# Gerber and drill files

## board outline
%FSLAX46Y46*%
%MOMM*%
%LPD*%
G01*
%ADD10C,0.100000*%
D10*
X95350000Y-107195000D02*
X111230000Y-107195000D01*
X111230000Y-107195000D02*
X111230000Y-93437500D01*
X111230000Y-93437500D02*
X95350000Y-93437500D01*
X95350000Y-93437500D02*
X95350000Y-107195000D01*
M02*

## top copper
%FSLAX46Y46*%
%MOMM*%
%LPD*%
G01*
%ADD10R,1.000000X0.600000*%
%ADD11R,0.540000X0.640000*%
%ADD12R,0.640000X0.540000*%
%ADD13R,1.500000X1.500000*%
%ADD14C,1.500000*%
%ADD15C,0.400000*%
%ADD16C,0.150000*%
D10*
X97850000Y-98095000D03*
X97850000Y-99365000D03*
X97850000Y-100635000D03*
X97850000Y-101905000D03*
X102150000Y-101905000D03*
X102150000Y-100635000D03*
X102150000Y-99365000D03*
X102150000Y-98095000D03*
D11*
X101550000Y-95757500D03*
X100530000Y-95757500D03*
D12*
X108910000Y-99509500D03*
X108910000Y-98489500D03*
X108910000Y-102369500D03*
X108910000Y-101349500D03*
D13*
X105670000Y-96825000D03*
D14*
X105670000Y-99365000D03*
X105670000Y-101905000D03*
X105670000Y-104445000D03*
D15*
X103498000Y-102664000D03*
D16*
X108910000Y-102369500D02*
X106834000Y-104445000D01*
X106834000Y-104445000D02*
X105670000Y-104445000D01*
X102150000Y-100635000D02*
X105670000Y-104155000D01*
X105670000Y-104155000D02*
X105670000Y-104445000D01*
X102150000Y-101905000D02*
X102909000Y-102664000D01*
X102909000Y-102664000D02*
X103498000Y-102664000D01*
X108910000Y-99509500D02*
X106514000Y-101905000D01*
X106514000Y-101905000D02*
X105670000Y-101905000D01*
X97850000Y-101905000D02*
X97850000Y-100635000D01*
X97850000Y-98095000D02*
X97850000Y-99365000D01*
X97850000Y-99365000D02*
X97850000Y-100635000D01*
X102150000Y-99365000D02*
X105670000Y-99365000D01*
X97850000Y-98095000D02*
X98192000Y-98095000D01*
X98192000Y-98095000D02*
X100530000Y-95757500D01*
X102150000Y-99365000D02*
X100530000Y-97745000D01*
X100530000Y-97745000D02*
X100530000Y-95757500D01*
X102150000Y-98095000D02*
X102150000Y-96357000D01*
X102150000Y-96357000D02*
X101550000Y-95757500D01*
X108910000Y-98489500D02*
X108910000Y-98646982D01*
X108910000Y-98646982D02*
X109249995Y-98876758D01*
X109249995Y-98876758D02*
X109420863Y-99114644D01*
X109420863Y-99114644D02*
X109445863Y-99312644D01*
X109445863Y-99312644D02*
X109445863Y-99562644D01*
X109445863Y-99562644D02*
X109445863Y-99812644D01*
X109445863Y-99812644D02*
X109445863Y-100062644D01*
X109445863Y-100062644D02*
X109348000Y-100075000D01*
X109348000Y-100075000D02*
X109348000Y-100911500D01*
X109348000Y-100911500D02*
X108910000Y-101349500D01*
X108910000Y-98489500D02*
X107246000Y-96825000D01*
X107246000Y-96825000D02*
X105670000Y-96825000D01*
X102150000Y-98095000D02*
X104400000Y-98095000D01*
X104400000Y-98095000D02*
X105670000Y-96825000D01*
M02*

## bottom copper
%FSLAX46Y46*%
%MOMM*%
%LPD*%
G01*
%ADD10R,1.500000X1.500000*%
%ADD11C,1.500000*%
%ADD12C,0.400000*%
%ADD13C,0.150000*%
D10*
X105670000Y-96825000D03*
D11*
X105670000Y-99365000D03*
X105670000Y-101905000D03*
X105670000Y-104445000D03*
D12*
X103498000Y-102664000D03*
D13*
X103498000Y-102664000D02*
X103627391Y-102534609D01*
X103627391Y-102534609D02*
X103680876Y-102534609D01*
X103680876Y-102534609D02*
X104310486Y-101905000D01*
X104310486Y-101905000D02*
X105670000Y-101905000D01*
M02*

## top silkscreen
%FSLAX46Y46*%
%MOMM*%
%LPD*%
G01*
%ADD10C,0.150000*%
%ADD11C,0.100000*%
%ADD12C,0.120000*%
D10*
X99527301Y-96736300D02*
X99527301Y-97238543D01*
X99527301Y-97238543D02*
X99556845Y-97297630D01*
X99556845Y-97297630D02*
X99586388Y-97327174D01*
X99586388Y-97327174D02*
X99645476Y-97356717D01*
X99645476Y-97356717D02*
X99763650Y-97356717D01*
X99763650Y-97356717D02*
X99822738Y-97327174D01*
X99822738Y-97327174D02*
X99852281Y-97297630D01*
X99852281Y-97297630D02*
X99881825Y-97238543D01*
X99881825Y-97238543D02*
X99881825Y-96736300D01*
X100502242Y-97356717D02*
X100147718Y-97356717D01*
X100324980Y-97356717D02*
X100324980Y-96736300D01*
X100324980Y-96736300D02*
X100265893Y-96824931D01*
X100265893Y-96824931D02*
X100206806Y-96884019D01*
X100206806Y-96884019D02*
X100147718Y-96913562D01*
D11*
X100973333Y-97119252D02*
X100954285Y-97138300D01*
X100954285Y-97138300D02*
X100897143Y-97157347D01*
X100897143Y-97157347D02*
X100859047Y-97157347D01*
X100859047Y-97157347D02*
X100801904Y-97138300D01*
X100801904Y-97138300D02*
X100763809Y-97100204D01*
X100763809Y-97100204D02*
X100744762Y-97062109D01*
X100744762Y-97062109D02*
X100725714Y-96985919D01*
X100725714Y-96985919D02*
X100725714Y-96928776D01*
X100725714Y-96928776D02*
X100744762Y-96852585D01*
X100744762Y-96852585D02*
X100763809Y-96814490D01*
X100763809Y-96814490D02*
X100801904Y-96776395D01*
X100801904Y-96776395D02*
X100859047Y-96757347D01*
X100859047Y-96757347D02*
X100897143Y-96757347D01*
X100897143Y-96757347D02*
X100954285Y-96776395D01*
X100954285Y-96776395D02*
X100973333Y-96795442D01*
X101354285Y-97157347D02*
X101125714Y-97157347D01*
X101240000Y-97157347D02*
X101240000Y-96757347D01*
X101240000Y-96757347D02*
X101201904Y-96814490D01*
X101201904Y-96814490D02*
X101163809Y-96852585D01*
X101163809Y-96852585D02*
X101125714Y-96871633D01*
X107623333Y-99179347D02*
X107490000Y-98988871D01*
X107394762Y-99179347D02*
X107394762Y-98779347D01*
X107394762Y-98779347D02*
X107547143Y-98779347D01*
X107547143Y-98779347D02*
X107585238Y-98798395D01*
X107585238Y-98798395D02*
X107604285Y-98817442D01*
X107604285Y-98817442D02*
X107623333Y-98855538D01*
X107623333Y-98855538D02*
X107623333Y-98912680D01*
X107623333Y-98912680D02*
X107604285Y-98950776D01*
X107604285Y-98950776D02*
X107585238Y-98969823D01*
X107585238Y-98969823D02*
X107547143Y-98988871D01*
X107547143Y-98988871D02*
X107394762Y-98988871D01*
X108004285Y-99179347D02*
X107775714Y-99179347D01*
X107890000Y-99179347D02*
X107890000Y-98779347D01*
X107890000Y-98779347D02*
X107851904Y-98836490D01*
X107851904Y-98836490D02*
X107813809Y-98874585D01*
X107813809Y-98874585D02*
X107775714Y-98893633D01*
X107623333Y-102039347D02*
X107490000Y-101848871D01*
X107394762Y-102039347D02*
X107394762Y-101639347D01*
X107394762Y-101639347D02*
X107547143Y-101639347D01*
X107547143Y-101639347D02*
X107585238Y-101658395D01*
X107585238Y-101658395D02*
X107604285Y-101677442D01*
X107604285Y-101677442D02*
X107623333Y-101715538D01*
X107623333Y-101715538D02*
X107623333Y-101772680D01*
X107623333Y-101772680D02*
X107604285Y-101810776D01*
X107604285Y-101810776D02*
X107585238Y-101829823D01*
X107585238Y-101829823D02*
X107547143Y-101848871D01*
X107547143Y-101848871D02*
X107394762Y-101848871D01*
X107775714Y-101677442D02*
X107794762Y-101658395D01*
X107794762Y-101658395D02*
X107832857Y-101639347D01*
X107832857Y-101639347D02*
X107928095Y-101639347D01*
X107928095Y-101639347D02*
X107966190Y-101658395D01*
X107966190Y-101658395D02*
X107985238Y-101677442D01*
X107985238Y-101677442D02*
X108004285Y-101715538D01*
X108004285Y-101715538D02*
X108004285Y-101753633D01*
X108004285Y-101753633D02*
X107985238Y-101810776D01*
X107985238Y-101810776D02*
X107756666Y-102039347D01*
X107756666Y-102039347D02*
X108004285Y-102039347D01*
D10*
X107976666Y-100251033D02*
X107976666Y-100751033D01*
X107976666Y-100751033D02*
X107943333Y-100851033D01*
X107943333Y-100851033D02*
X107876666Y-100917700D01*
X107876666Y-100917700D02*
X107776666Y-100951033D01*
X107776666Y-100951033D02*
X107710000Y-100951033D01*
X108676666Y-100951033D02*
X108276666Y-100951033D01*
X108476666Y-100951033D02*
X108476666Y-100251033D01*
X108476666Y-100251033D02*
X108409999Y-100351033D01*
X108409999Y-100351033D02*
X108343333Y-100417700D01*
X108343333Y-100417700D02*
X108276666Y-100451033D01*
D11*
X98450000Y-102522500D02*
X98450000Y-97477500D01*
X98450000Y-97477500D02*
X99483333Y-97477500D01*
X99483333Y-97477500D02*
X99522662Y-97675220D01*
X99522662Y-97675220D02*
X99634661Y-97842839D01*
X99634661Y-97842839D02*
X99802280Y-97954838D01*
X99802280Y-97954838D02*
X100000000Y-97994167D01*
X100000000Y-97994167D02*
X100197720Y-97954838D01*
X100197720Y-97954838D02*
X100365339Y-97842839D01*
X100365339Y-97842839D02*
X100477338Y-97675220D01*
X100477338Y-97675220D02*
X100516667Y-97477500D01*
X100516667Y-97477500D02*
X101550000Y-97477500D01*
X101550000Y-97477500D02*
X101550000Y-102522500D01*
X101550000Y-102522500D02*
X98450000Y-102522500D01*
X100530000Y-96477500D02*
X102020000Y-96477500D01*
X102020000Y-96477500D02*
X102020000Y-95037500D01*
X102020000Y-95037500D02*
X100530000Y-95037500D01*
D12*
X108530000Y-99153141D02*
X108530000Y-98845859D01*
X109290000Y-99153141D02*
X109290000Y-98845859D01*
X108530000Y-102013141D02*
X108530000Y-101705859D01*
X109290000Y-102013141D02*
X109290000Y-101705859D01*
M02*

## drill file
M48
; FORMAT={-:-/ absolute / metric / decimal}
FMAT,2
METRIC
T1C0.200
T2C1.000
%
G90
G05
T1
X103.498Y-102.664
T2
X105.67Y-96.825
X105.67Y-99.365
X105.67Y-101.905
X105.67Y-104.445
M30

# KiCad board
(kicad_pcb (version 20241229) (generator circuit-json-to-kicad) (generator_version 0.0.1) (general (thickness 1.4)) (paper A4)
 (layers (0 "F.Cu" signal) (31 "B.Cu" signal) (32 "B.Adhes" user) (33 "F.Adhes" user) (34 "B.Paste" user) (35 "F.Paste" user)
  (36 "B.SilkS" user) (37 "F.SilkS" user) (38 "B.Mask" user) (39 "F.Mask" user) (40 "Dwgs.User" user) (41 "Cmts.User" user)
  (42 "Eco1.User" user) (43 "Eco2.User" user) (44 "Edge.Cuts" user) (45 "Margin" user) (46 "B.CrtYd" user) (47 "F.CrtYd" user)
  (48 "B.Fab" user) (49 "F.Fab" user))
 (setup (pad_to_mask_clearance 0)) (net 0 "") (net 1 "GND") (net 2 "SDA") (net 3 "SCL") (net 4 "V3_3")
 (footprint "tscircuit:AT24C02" (layer F.Cu) (at 100 100 0)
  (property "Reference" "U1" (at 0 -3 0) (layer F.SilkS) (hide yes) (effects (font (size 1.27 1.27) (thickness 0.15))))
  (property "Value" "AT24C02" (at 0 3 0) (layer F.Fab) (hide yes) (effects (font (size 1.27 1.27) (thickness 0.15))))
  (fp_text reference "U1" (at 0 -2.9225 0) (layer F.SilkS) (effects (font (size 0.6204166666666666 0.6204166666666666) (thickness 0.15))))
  (fp_line (start -1.5499999999999998 2.5225) (end -1.5499999999999998 -2.5225) (stroke (width 0.1) (type default)) (layer F.SilkS))
  (fp_line (start -1.5499999999999998 -2.5225) (end -0.5166666666666666 -2.5225) (stroke (width 0.1) (type default)) (layer F.SilkS))
  (fp_line (start -0.5166666666666666 -2.5225) (end -0.47733775846416476 -2.32478022661137) (stroke (width 0.1) (type default))
   (layer F.SilkS))
  (fp_line (start -0.47733775846416476 -2.32478022661137) (end -0.3653385036130495 -2.1571614963869505) (stroke (width 0.1) (type default))
   (layer F.SilkS))
  (fp_line (start -0.3653385036130495 -2.1571614963869505) (end -0.19771977338862967 -2.0451622415358353)
   (stroke (width 0.1) (type default)) (layer F.SilkS))
  (fp_line (start -0.19771977338862967 -2.0451622415358353) (end 3.1636708977973285e-17 -2.0058333333333334)
   (stroke (width 0.1) (type default)) (layer F.SilkS))
  (fp_line (start 3.1636708977973285e-17 -2.0058333333333334) (end 0.1977197733886297 -2.0451622415358353)
   (stroke (width 0.1) (type default)) (layer F.SilkS))
  (fp_line (start 0.1977197733886297 -2.0451622415358353) (end 0.3653385036130496 -2.1571614963869505) (stroke (width 0.1) (type default))
   (layer F.SilkS))
  (fp_line (start 0.3653385036130496 -2.1571614963869505) (end 0.47733775846416476 -2.32478022661137) (stroke (width 0.1) (type default))
   (layer F.SilkS))
  (fp_line (start 0.47733775846416476 -2.32478022661137) (end 0.5166666666666666 -2.5225) (stroke (width 0.1) (type default))
   (layer F.SilkS))
  (fp_line (start 0.5166666666666666 -2.5225) (end 1.5499999999999998 -2.5225) (stroke (width 0.1) (type default)) (layer F.SilkS))
  (fp_line (start 1.5499999999999998 -2.5225) (end 1.5499999999999998 2.5225) (stroke (width 0.1) (type default)) (layer F.SilkS))
  (fp_line (start 1.5499999999999998 2.5225) (end -1.5499999999999998 2.5225) (stroke (width 0.1) (type default)) (layer F.SilkS))
  (pad "1" smd rect (at -2.15 -1.905 0) (size 1 0.6) (layers F.Cu F.Paste F.Mask) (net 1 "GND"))
  (pad "2" smd rect (at -2.15 -0.635 0) (size 1 0.6) (layers F.Cu F.Paste F.Mask) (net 1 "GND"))
  (pad "3" smd rect (at -2.15 0.635 0) (size 1 0.6) (layers F.Cu F.Paste F.Mask) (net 1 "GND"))
  (pad "4" smd rect (at -2.15 1.905 0) (size 1 0.6) (layers F.Cu F.Paste F.Mask) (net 1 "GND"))
  (pad "5" smd rect (at 2.15 1.905 0) (size 1 0.6) (layers F.Cu F.Paste F.Mask) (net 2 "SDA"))
  (pad "6" smd rect (at 2.15 0.635 0) (size 1 0.6) (layers F.Cu F.Paste F.Mask) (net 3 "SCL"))
  (pad "7" smd rect (at 2.15 -0.635 0) (size 1 0.6) (layers F.Cu F.Paste F.Mask) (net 1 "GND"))
  (pad "8" smd rect (at 2.15 -1.905 0) (size 1 0.6) (layers F.Cu F.Paste F.Mask) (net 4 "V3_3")))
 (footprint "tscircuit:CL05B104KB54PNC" (layer F.Cu) (at 101.04 95.7575 180)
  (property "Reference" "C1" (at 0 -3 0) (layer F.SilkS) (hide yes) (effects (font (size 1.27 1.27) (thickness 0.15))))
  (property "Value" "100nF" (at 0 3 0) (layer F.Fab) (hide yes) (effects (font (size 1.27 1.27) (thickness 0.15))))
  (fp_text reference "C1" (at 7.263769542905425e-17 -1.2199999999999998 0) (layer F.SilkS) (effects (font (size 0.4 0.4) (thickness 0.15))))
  (fp_line (start 0.51 -0.7199999999999999) (end -0.9800000000000001 -0.7200000000000001) (stroke (width 0.1) (type default))
   (layer F.SilkS))
  (fp_line (start -0.9800000000000001 -0.7200000000000001) (end -0.9799999999999999 0.7199999999999999) (stroke (width 0.1) (type default))
   (layer F.SilkS))
  (fp_line (start -0.9799999999999999 0.7199999999999999) (end 0.51 0.7199999999999996) (stroke (width 0.1) (type default)) (layer F.SilkS))
  (pad "1" smd rect (at -0.51 0 0) (size 0.54 0.64) (layers F.Cu F.Paste F.Mask) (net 4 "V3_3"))
  (pad "2" smd rect (at 0.5100000000000001 0 0) (size 0.54 0.64) (layers F.Cu F.Paste F.Mask) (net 1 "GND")))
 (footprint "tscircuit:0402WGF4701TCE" (layer F.Cu) (at 108.91 98.9995 90)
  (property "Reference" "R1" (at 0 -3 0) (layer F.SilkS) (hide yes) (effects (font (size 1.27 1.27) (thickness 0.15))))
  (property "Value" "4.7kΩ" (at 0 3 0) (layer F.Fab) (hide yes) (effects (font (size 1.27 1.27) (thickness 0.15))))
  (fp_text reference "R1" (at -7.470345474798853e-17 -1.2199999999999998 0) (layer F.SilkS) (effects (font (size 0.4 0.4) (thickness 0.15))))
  (fp_line (start -0.15364099999999994 -0.3800000000000008) (end 0.1536409999999999 -0.3800000000000008)
   (stroke (width 0.12) (type default)) (layer F.SilkS))
  (fp_line (start -0.153641 0.3800000000000008) (end 0.15364099999999994 0.3800000000000008) (stroke (width 0.12) (type default))
   (layer F.SilkS))
  (pad "1" smd rect (at -0.5099999999999999 0 0) (size 0.64 0.54) (layers F.Cu F.Paste F.Mask) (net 2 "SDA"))
  (pad "2" smd rect (at 0.51 0 0) (size 0.64 0.54) (layers F.Cu F.Paste F.Mask) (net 4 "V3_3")))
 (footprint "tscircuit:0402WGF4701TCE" (layer F.Cu) (at 108.91 101.8595 90)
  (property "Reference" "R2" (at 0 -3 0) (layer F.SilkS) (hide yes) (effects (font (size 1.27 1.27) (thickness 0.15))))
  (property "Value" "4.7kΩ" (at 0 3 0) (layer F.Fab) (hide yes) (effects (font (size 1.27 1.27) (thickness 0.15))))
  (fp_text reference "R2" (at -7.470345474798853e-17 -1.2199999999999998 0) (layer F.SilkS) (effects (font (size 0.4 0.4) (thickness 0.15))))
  (fp_line (start -0.15364099999999994 -0.3800000000000008) (end 0.1536409999999999 -0.3800000000000008)
   (stroke (width 0.12) (type default)) (layer F.SilkS))
  (fp_line (start -0.1536409999999999 0.3800000000000008) (end 0.15364099999999994 0.3800000000000008) (stroke (width 0.12) (type default))
   (layer F.SilkS))
  (pad "1" smd rect (at -0.5099999999999998 0 0) (size 0.64 0.54) (layers F.Cu F.Paste F.Mask) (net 3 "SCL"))
  (pad "2" smd rect (at 0.51 0 0) (size 0.64 0.54) (layers F.Cu F.Paste F.Mask) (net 4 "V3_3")))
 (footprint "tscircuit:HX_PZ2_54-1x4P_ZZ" (layer F.Cu) (at 105.67 100.635 -90.00000000000001)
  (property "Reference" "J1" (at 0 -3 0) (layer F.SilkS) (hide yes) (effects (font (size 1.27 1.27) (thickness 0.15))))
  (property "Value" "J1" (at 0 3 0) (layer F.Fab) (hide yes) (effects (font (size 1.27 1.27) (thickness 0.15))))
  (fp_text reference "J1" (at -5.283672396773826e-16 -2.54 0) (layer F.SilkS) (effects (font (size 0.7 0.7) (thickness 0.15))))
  (pad "1" thru_hole rect (at -3.81 5.705062545910424e-16 0) (size 1.5 1.5) (drill 1) (layers *.Cu *.Mask) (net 4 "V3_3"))
  (pad "2" thru_hole circle (at -1.27 4.862282247637226e-16 0) (size 1.5 1.5) (drill 1) (layers *.Cu *.Mask) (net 1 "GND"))
  (pad "3" thru_hole circle (at 1.27 -4.862282247637226e-16 0) (size 1.5 1.5) (drill 1) (layers *.Cu *.Mask) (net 2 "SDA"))
  (pad "4" thru_hole circle (at 3.8100000000000005 -5.705062545910426e-16 0) (size 1.5 1.5) (drill 1) (layers *.Cu *.Mask) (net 3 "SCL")))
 (segment (start 108.91 102.3695) (end 106.834 104.44500000000001) (width 0.15) (layer F.Cu) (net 3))
 (segment (start 106.834 104.44500000000001) (end 105.67 104.44500000000001) (width 0.15) (layer F.Cu) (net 3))
 (segment (start 102.15 100.635) (end 105.67 104.155) (width 0.15) (layer F.Cu) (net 3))
 (segment (start 105.67 104.155) (end 105.67 104.44500000000001) (width 0.15) (layer F.Cu) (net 3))
 (segment (start 102.15 101.905) (end 102.909 102.664) (width 0.15) (layer F.Cu) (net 2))
 (segment (start 102.909 102.664) (end 103.498 102.664) (width 0.15) (layer F.Cu) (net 2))
 (segment (start 103.498 102.664) (end 103.62739082395659 102.53460917604342) (width 0.15) (layer B.Cu) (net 2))
 (segment (start 103.62739082395659 102.53460917604342) (end 103.68087635753074 102.53460917604342) (width 0.15) (layer B.Cu) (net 2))
 (segment (start 103.68087635753074 102.53460917604342) (end 104.31048553357415 101.905) (width 0.15) (layer B.Cu) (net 2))
 (segment (start 104.31048553357415 101.905) (end 105.67 101.905) (width 0.15) (layer B.Cu) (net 2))
 (segment (start 108.91 99.5095) (end 106.514 101.905) (width 0.15) (layer F.Cu) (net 2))
 (segment (start 106.514 101.905) (end 105.67 101.905) (width 0.15) (layer F.Cu) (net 2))
 (segment (start 97.85 101.905) (end 97.85 100.635) (width 0.15) (layer F.Cu) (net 1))
 (segment (start 97.85 98.095) (end 97.85 99.365) (width 0.15) (layer F.Cu) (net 1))
 (segment (start 97.85 99.365) (end 97.85 100.635) (width 0.15) (layer F.Cu) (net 1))
 (segment (start 102.15 99.365) (end 105.67 99.365) (width 0.15) (layer F.Cu) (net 1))
 (segment (start 97.85 98.095) (end 98.192 98.095) (width 0.15) (layer F.Cu) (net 1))
 (segment (start 98.192 98.095) (end 100.53 95.7575) (width 0.15) (layer F.Cu) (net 1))
 (segment (start 102.15 99.365) (end 100.53 97.745) (width 0.15) (layer F.Cu) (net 1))
 (segment (start 100.53 97.745) (end 100.53 95.7575) (width 0.15) (layer F.Cu) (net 1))
 (segment (start 102.15 98.095) (end 102.15 96.357) (width 0.15) (layer F.Cu) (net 4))
 (segment (start 102.15 96.357) (end 101.55 95.7575) (width 0.15) (layer F.Cu) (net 4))
 (segment (start 108.91 98.48949999999999) (end 108.91 98.64698194937783) (width 0.15) (layer F.Cu) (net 4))
 (segment (start 108.91 98.64698194937783) (end 109.24999537270699 98.87675797422321) (width 0.15) (layer F.Cu) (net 4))
 (segment (start 109.24999537270699 98.87675797422321) (end 109.42086291872914 99.11464357086753) (width 0.15) (layer F.Cu) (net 4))
 (segment (start 109.42086291872914 99.11464357086753) (end 109.44586291872915 99.31264357086754) (width 0.15) (layer F.Cu) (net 4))
 (segment (start 109.44586291872915 99.31264357086754) (end 109.44586291872915 99.56264357086754) (width 0.15) (layer F.Cu) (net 4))
 (segment (start 109.44586291872915 99.56264357086754) (end 109.44586291872915 99.81264357086754) (width 0.15) (layer F.Cu) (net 4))
 (segment (start 109.44586291872915 99.81264357086754) (end 109.44586291872915 100.06264357086754) (width 0.15) (layer F.Cu) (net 4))
 (segment (start 109.44586291872915 100.06264357086754) (end 109.348 100.075) (width 0.15) (layer F.Cu) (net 4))
 (segment (start 109.348 100.075) (end 109.348 100.9115) (width 0.15) (layer F.Cu) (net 4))
 (segment (start 109.348 100.9115) (end 108.91 101.3495) (width 0.15) (layer F.Cu) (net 4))
 (segment (start 108.91 98.48949999999999) (end 107.246 96.825) (width 0.15) (layer F.Cu) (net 4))
 (segment (start 107.246 96.825) (end 105.67 96.825) (width 0.15) (layer F.Cu) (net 4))
 (segment (start 102.15 98.095) (end 104.4 98.095) (width 0.15) (layer F.Cu) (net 4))
 (segment (start 104.4 98.095) (end 105.67 96.825) (width 0.15) (layer F.Cu) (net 4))
 (gr_line (start 95.35 107.19500000000001) (end 111.23 107.19500000000001) (width 0.1) (layer Edge.Cuts))
 (gr_line (start 111.23 107.19500000000001) (end 111.23 93.4375) (width 0.1) (layer Edge.Cuts))
 (gr_line (start 111.23 93.4375) (end 95.35 93.4375) (width 0.1) (layer Edge.Cuts))
 (gr_line (start 95.35 93.4375) (end 95.35 107.19500000000001) (width 0.1) (layer Edge.Cuts))
 (via (at 103.498 102.664) (size 0.4) (drill 0.2) (layers F.Cu B.Cu) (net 2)))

